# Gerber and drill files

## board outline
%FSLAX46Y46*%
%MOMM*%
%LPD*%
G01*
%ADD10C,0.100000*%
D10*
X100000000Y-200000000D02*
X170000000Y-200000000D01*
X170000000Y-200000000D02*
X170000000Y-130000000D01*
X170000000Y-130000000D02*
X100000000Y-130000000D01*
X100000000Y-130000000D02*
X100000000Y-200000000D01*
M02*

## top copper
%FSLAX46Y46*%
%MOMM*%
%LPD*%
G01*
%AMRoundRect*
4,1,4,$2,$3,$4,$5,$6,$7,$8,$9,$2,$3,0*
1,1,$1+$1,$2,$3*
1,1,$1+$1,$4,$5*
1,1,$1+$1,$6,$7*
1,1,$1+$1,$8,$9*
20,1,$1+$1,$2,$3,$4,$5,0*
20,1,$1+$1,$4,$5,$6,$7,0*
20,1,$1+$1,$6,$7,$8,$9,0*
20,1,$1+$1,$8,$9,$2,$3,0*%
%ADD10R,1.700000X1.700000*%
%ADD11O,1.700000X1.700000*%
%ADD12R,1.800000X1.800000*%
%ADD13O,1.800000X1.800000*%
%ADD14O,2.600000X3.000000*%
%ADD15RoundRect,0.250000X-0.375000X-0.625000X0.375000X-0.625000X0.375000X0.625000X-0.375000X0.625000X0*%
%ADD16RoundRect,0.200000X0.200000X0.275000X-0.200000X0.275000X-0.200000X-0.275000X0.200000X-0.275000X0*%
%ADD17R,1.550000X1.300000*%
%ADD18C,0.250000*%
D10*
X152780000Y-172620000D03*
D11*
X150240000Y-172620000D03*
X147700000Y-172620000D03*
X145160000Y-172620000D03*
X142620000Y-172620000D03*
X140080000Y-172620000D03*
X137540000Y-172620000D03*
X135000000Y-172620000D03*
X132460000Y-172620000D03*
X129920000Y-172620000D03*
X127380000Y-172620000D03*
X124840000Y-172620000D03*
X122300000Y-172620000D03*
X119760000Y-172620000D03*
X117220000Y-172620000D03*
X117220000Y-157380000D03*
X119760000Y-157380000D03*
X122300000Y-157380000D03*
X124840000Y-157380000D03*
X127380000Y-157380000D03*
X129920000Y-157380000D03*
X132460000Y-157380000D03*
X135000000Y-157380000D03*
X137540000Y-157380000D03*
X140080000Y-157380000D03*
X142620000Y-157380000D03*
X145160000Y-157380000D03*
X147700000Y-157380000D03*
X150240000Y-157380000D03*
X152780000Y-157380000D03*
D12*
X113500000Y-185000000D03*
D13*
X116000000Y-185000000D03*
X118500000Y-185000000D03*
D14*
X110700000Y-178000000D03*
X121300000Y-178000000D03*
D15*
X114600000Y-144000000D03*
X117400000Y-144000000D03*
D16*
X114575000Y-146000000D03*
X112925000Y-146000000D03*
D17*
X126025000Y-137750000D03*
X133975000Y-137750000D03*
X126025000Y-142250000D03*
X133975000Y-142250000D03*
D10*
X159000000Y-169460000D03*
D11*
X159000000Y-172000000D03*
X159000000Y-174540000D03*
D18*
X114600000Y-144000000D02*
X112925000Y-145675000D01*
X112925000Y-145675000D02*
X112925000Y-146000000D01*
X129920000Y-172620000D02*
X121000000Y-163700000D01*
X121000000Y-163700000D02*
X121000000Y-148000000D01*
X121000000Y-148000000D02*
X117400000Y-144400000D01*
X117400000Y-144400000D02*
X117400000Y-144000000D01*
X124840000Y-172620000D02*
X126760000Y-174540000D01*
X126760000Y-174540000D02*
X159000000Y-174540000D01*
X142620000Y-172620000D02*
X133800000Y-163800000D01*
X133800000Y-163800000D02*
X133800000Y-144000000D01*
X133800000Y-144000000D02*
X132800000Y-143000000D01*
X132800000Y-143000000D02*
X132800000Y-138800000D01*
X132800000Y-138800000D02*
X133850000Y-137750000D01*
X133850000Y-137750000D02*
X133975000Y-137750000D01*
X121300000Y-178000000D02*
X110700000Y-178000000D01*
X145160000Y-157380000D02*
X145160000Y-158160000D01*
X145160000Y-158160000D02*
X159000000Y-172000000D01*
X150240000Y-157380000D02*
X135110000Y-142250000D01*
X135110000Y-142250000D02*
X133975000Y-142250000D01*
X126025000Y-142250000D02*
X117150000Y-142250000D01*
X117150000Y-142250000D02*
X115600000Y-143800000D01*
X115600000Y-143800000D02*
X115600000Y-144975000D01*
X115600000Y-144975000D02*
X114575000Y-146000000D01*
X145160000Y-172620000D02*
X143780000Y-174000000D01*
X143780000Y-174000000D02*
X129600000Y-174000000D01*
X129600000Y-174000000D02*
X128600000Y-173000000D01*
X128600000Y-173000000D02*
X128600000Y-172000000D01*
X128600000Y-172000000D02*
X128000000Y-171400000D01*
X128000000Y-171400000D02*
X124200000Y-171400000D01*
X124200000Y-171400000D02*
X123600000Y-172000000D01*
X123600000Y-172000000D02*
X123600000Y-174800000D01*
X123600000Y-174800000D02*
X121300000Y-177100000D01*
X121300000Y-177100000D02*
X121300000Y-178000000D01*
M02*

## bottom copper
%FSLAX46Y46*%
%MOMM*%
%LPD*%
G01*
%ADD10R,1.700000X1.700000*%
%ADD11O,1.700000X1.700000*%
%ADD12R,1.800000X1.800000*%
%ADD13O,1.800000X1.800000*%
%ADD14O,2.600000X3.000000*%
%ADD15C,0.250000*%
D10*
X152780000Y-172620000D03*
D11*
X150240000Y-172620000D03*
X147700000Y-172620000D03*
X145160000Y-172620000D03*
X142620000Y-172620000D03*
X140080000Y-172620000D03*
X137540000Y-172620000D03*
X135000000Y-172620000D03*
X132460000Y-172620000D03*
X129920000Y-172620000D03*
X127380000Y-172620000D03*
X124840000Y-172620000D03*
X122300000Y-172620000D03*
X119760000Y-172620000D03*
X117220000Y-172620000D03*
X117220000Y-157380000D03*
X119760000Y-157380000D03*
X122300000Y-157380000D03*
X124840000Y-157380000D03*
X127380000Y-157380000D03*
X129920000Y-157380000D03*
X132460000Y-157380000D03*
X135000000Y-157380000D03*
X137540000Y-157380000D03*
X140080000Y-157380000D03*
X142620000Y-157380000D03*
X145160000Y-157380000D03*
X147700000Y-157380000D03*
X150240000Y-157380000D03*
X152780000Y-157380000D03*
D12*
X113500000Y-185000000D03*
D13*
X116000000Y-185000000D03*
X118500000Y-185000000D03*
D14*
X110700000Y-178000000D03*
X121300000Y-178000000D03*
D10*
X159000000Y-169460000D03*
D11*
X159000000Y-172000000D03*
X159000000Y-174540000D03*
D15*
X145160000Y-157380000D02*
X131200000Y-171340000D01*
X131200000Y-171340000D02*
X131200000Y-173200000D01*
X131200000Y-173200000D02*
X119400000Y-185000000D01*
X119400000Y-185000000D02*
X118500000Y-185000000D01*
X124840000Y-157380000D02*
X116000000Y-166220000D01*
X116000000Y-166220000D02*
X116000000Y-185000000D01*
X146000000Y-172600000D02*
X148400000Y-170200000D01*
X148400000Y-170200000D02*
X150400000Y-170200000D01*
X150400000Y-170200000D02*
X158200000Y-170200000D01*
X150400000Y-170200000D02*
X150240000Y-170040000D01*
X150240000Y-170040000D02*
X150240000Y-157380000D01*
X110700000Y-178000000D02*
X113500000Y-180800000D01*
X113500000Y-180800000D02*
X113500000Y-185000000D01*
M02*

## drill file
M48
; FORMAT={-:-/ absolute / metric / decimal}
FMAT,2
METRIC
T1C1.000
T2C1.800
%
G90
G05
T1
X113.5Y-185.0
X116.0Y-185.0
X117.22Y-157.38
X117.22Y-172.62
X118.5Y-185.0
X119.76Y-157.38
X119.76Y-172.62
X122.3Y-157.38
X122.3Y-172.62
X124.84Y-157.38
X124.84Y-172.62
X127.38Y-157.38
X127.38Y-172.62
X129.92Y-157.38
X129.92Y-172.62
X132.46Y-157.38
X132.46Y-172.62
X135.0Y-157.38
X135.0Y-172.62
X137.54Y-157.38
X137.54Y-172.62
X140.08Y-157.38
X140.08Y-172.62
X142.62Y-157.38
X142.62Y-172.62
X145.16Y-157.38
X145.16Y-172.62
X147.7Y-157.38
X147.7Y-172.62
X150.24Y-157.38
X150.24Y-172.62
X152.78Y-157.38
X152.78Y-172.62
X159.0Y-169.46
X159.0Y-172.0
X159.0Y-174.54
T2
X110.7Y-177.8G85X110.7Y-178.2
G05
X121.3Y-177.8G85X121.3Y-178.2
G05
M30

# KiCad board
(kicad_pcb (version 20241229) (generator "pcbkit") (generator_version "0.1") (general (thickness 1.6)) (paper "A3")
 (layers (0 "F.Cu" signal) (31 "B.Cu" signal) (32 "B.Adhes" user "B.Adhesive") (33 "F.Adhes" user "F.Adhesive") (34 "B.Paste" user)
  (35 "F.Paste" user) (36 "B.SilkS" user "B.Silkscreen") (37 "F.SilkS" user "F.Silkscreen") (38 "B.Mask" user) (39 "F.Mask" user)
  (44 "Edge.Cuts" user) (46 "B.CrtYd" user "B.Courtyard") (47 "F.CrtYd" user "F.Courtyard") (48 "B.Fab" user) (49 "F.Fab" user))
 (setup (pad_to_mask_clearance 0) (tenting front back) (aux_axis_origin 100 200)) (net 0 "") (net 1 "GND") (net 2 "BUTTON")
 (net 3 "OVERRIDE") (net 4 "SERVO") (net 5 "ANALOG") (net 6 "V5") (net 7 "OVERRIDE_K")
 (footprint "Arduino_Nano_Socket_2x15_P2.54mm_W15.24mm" (layer "B.Cu") (at 135 165 90)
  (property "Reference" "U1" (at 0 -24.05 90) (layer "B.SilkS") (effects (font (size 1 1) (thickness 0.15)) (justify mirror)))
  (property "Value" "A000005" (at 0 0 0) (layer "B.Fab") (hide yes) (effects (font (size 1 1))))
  (pad "1" thru_hole rect (at -7.62 17.78 90) (size 1.7 1.7) (drill 1) (layers "*.Cu" "*.Mask") (solder_mask_margin 0.05))
  (pad "2" thru_hole oval (at -7.62 15.24 90) (size 1.7 1.7) (drill 1) (layers "*.Cu" "*.Mask") (solder_mask_margin 0.05))
  (pad "3" thru_hole oval (at -7.62 12.7 90) (size 1.7 1.7) (drill 1) (layers "*.Cu" "*.Mask") (solder_mask_margin 0.05))
  (pad "4" thru_hole oval (at -7.62 10.16 90) (size 1.7 1.7) (drill 1) (layers "*.Cu" "*.Mask") (solder_mask_margin 0.05) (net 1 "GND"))
  (pad "5" thru_hole oval (at -7.62 7.62 90) (size 1.7 1.7) (drill 1) (layers "*.Cu" "*.Mask") (solder_mask_margin 0.05) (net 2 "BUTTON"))
  (pad "6" thru_hole oval (at -7.62 5.08 90) (size 1.7 1.7) (drill 1) (layers "*.Cu" "*.Mask") (solder_mask_margin 0.05))
  (pad "7" thru_hole oval (at -7.62 2.54 90) (size 1.7 1.7) (drill 1) (layers "*.Cu" "*.Mask") (solder_mask_margin 0.05))
  (pad "8" thru_hole oval (at -7.62 0 90) (size 1.7 1.7) (drill 1) (layers "*.Cu" "*.Mask") (solder_mask_margin 0.05))
  (pad "9" thru_hole oval (at -7.62 -2.54 90) (size 1.7 1.7) (drill 1) (layers "*.Cu" "*.Mask") (solder_mask_margin 0.05))
  (pad "10" thru_hole oval (at -7.62 -5.08 90) (size 1.7 1.7) (drill 1) (layers "*.Cu" "*.Mask") (solder_mask_margin 0.05)
   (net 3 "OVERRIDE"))
  (pad "11" thru_hole oval (at -7.62 -7.62 90) (size 1.7 1.7) (drill 1) (layers "*.Cu" "*.Mask") (solder_mask_margin 0.05))
  (pad "12" thru_hole oval (at -7.62 -10.16 90) (size 1.7 1.7) (drill 1) (layers "*.Cu" "*.Mask") (solder_mask_margin 0.05) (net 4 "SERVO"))
  (pad "13" thru_hole oval (at -7.62 -12.7 90) (size 1.7 1.7) (drill 1) (layers "*.Cu" "*.Mask") (solder_mask_margin 0.05))
  (pad "14" thru_hole oval (at -7.62 -15.24 90) (size 1.7 1.7) (drill 1) (layers "*.Cu" "*.Mask") (solder_mask_margin 0.05))
  (pad "15" thru_hole oval (at -7.62 -17.78 90) (size 1.7 1.7) (drill 1) (layers "*.Cu" "*.Mask") (solder_mask_margin 0.05))
  (pad "16" thru_hole oval (at 7.62 -17.78 90) (size 1.7 1.7) (drill 1) (layers "*.Cu" "*.Mask") (solder_mask_margin 0.05))
  (pad "17" thru_hole oval (at 7.62 -15.24 90) (size 1.7 1.7) (drill 1) (layers "*.Cu" "*.Mask") (solder_mask_margin 0.05))
  (pad "18" thru_hole oval (at 7.62 -12.7 90) (size 1.7 1.7) (drill 1) (layers "*.Cu" "*.Mask") (solder_mask_margin 0.05))
  (pad "19" thru_hole oval (at 7.62 -10.16 90) (size 1.7 1.7) (drill 1) (layers "*.Cu" "*.Mask") (solder_mask_margin 0.05) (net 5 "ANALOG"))
  (pad "20" thru_hole oval (at 7.62 -7.62 90) (size 1.7 1.7) (drill 1) (layers "*.Cu" "*.Mask") (solder_mask_margin 0.05))
  (pad "21" thru_hole oval (at 7.62 -5.08 90) (size 1.7 1.7) (drill 1) (layers "*.Cu" "*.Mask") (solder_mask_margin 0.05))
  (pad "22" thru_hole oval (at 7.62 -2.54 90) (size 1.7 1.7) (drill 1) (layers "*.Cu" "*.Mask") (solder_mask_margin 0.05))
  (pad "23" thru_hole oval (at 7.62 0 90) (size 1.7 1.7) (drill 1) (layers "*.Cu" "*.Mask") (solder_mask_margin 0.05))
  (pad "24" thru_hole oval (at 7.62 2.54 90) (size 1.7 1.7) (drill 1) (layers "*.Cu" "*.Mask") (solder_mask_margin 0.05))
  (pad "25" thru_hole oval (at 7.62 5.08 90) (size 1.7 1.7) (drill 1) (layers "*.Cu" "*.Mask") (solder_mask_margin 0.05))
  (pad "26" thru_hole oval (at 7.62 7.62 90) (size 1.7 1.7) (drill 1) (layers "*.Cu" "*.Mask") (solder_mask_margin 0.05))
  (pad "27" thru_hole oval (at 7.62 10.16 90) (size 1.7 1.7) (drill 1) (layers "*.Cu" "*.Mask") (solder_mask_margin 0.05) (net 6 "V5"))
  (pad "28" thru_hole oval (at 7.62 12.7 90) (size 1.7 1.7) (drill 1) (layers "*.Cu" "*.Mask") (solder_mask_margin 0.05))
  (pad "29" thru_hole oval (at 7.62 15.24 90) (size 1.7 1.7) (drill 1) (layers "*.Cu" "*.Mask") (solder_mask_margin 0.05) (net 1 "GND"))
  (pad "30" thru_hole oval (at 7.62 17.78 90) (size 1.7 1.7) (drill 1) (layers "*.Cu" "*.Mask") (solder_mask_margin 0.05)))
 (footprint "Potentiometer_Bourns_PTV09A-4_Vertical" (layer "F.Cu") (at 116 185 0)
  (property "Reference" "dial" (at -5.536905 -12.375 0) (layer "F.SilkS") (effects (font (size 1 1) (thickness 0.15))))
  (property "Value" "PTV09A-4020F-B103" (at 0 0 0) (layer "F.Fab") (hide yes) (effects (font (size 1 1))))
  (pad "1" thru_hole rect (at -2.5 0 0) (size 1.8 1.8) (drill 1) (layers "*.Cu" "*.Mask") (solder_mask_margin 0.05) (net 1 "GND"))
  (pad "2" thru_hole oval (at 0 0 0) (size 1.8 1.8) (drill 1) (layers "*.Cu" "*.Mask") (solder_mask_margin 0.05) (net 5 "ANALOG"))
  (pad "3" thru_hole oval (at 2.5 0 0) (size 1.8 1.8) (drill 1) (layers "*.Cu" "*.Mask") (solder_mask_margin 0.05) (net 6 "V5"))
  (pad "MP" thru_hole oval (at -5.3 -7 0) (size 2.6 3) (drill oval 1.8 2.2) (layers "*.Cu" "*.Mask") (solder_mask_margin 0.05) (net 1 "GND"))
  (pad "MP" thru_hole oval (at 5.3 -7 0) (size 2.6 3) (drill oval 1.8 2.2) (layers "*.Cu" "*.Mask") (solder_mask_margin 0.05) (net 1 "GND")))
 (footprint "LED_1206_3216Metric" (layer "F.Cu") (at 116 144 0)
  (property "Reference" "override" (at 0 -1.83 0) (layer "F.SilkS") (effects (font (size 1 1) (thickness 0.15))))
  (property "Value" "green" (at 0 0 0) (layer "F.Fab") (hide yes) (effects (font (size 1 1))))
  (pad "1" smd roundrect (at -1.4 0 0) (size 1.25 1.75) (layers "F.Cu" "F.Paste" "F.Mask") (roundrect_rratio 0.200000000000)
   (solder_mask_margin 0.05) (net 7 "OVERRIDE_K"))
  (pad "2" smd roundrect (at 1.4 0 0) (size 1.25 1.75) (layers "F.Cu" "F.Paste" "F.Mask") (roundrect_rratio 0.200000000000)
   (solder_mask_margin 0.05) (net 3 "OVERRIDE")))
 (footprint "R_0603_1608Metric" (layer "F.Cu") (at 113.75 146 180)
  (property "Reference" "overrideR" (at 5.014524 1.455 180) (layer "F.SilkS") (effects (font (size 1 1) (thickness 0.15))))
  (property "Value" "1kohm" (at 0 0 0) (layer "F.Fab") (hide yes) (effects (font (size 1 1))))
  (pad "1" smd roundrect (at -0.825 0 180) (size 0.8 0.95) (layers "F.Cu" "F.Paste" "F.Mask") (roundrect_rratio 0.250000000000)
   (solder_mask_margin 0.05) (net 1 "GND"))
  (pad "2" smd roundrect (at 0.825 0 180) (size 0.8 0.95) (layers "F.Cu" "F.Paste" "F.Mask") (roundrect_rratio 0.250000000000)
   (solder_mask_margin 0.05) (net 7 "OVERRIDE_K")))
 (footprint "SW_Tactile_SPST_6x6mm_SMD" (layer "F.Cu") (at 130 140 0)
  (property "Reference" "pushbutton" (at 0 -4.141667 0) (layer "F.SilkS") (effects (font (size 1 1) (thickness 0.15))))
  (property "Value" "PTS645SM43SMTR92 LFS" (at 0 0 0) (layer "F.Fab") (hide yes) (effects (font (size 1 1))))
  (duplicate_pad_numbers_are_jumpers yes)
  (pad "1" smd rect (at -3.975 -2.25 0) (size 1.55 1.3) (layers "F.Cu" "F.Paste" "F.Mask") (solder_mask_margin 0.05) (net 2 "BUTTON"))
  (pad "1" smd rect (at 3.975 -2.25 0) (size 1.55 1.3) (layers "F.Cu" "F.Paste" "F.Mask") (solder_mask_margin 0.05) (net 2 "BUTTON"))
  (pad "2" smd rect (at -3.975 2.25 0) (size 1.55 1.3) (layers "F.Cu" "F.Paste" "F.Mask") (solder_mask_margin 0.05) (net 1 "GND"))
  (pad "2" smd rect (at 3.975 2.25 0) (size 1.55 1.3) (layers "F.Cu" "F.Paste" "F.Mask") (solder_mask_margin 0.05) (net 1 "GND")))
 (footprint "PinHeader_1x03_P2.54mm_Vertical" (layer "F.Cu") (at 159 172 0)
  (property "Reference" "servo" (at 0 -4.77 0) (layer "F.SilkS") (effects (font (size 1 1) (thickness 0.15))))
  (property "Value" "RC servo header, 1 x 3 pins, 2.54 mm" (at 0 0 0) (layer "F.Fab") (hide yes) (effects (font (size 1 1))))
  (pad "1" thru_hole rect (at 0 -2.54 0) (size 1.7 1.7) (drill 1) (layers "*.Cu" "*.Mask") (solder_mask_margin 0.05) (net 1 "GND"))
  (pad "2" thru_hole oval (at 0 0 0) (size 1.7 1.7) (drill 1) (layers "*.Cu" "*.Mask") (solder_mask_margin 0.05) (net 6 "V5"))
  (pad "3" thru_hole oval (at 0 2.54 0) (size 1.7 1.7) (drill 1) (layers "*.Cu" "*.Mask") (solder_mask_margin 0.05) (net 4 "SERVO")))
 (segment (start 114.6 144) (end 112.925 145.675) (width 0.25) (layer "F.Cu") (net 7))
 (segment (start 112.925 145.675) (end 112.925 146) (width 0.25) (layer "F.Cu") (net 7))
 (segment (start 129.92 172.62) (end 121 163.7) (width 0.25) (layer "F.Cu") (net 3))
 (segment (start 121 163.7) (end 121 148) (width 0.25) (layer "F.Cu") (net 3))
 (segment (start 121 148) (end 117.4 144.4) (width 0.25) (layer "F.Cu") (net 3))
 (segment (start 117.4 144.4) (end 117.4 144) (width 0.25) (layer "F.Cu") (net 3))
 (segment (start 124.84 172.62) (end 126.76 174.54) (width 0.25) (layer "F.Cu") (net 4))
 (segment (start 126.76 174.54) (end 159 174.54) (width 0.25) (layer "F.Cu") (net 4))
 (segment (start 142.62 172.62) (end 133.8 163.8) (width 0.25) (layer "F.Cu") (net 2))
 (segment (start 133.8 163.8) (end 133.8 144) (width 0.25) (layer "F.Cu") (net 2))
 (segment (start 133.8 144) (end 132.8 143) (width 0.25) (layer "F.Cu") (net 2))
 (segment (start 132.8 143) (end 132.8 138.8) (width 0.25) (layer "F.Cu") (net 2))
 (segment (start 132.8 138.8) (end 133.85 137.75) (width 0.25) (layer "F.Cu") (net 2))
 (segment (start 133.85 137.75) (end 133.975 137.75) (width 0.25) (layer "F.Cu") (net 2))
 (segment (start 121.3 178) (end 110.7 178) (width 0.25) (layer "F.Cu") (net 1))
 (segment (start 145.16 157.38) (end 145.16 158.16) (width 0.25) (layer "F.Cu") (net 6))
 (segment (start 145.16 158.16) (end 159 172) (width 0.25) (layer "F.Cu") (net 6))
 (segment (start 145.16 157.38) (end 131.2 171.34) (width 0.25) (layer "B.Cu") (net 6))
 (segment (start 131.2 171.34) (end 131.2 173.2) (width 0.25) (layer "B.Cu") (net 6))
 (segment (start 131.2 173.2) (end 119.4 185) (width 0.25) (layer "B.Cu") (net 6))
 (segment (start 119.4 185) (end 118.5 185) (width 0.25) (layer "B.Cu") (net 6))
 (segment (start 124.84 157.38) (end 116 166.22) (width 0.25) (layer "B.Cu") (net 5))
 (segment (start 116 166.22) (end 116 185) (width 0.25) (layer "B.Cu") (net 5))
 (segment (start 146 172.6) (end 148.4 170.2) (width 0.25) (layer "B.Cu") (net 1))
 (segment (start 148.4 170.2) (end 150.4 170.2) (width 0.25) (layer "B.Cu") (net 1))
 (segment (start 150.4 170.2) (end 158.2 170.2) (width 0.25) (layer "B.Cu") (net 1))
 (segment (start 150.4 170.2) (end 150.24 170.04) (width 0.25) (layer "B.Cu") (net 1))
 (segment (start 150.24 170.04) (end 150.24 157.38) (width 0.25) (layer "B.Cu") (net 1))
 (segment (start 150.24 157.38) (end 135.11 142.25) (width 0.25) (layer "F.Cu") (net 1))
 (segment (start 135.11 142.25) (end 133.975 142.25) (width 0.25) (layer "F.Cu") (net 1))
 (segment (start 126.025 142.25) (end 117.15 142.25) (width 0.25) (layer "F.Cu") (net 1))
 (segment (start 117.15 142.25) (end 115.6 143.8) (width 0.25) (layer "F.Cu") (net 1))
 (segment (start 115.6 143.8) (end 115.6 144.975) (width 0.25) (layer "F.Cu") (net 1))
 (segment (start 115.6 144.975) (end 114.575 146) (width 0.25) (layer "F.Cu") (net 1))
 (segment (start 145.16 172.62) (end 143.78 174) (width 0.25) (layer "F.Cu") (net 1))
 (segment (start 143.78 174) (end 129.6 174) (width 0.25) (layer "F.Cu") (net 1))
 (segment (start 129.6 174) (end 128.6 173) (width 0.25) (layer "F.Cu") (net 1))
 (segment (start 128.6 173) (end 128.6 172) (width 0.25) (layer "F.Cu") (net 1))
 (segment (start 128.6 172) (end 128 171.4) (width 0.25) (layer "F.Cu") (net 1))
 (segment (start 128 171.4) (end 124.2 171.4) (width 0.25) (layer "F.Cu") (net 1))
 (segment (start 124.2 171.4) (end 123.6 172) (width 0.25) (layer "F.Cu") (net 1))
 (segment (start 123.6 172) (end 123.6 174.8) (width 0.25) (layer "F.Cu") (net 1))
 (segment (start 123.6 174.8) (end 121.3 177.1) (width 0.25) (layer "F.Cu") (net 1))
 (segment (start 121.3 177.1) (end 121.3 178) (width 0.25) (layer "F.Cu") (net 1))
 (segment (start 110.7 178) (end 113.5 180.8) (width 0.25) (layer "B.Cu") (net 1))
 (segment (start 113.5 180.8) (end 113.5 185) (width 0.25) (layer "B.Cu") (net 1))
 (gr_line (start 100 200) (end 170 200) (stroke (width 0.1) (type solid)) (layer "Edge.Cuts"))
 (gr_line (start 170 200) (end 170 130) (stroke (width 0.1) (type solid)) (layer "Edge.Cuts"))
 (gr_line (start 170 130) (end 100 130) (stroke (width 0.1) (type solid)) (layer "Edge.Cuts"))
 (gr_line (start 100 130) (end 100 200) (stroke (width 0.1) (type solid)) (layer "Edge.Cuts")))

